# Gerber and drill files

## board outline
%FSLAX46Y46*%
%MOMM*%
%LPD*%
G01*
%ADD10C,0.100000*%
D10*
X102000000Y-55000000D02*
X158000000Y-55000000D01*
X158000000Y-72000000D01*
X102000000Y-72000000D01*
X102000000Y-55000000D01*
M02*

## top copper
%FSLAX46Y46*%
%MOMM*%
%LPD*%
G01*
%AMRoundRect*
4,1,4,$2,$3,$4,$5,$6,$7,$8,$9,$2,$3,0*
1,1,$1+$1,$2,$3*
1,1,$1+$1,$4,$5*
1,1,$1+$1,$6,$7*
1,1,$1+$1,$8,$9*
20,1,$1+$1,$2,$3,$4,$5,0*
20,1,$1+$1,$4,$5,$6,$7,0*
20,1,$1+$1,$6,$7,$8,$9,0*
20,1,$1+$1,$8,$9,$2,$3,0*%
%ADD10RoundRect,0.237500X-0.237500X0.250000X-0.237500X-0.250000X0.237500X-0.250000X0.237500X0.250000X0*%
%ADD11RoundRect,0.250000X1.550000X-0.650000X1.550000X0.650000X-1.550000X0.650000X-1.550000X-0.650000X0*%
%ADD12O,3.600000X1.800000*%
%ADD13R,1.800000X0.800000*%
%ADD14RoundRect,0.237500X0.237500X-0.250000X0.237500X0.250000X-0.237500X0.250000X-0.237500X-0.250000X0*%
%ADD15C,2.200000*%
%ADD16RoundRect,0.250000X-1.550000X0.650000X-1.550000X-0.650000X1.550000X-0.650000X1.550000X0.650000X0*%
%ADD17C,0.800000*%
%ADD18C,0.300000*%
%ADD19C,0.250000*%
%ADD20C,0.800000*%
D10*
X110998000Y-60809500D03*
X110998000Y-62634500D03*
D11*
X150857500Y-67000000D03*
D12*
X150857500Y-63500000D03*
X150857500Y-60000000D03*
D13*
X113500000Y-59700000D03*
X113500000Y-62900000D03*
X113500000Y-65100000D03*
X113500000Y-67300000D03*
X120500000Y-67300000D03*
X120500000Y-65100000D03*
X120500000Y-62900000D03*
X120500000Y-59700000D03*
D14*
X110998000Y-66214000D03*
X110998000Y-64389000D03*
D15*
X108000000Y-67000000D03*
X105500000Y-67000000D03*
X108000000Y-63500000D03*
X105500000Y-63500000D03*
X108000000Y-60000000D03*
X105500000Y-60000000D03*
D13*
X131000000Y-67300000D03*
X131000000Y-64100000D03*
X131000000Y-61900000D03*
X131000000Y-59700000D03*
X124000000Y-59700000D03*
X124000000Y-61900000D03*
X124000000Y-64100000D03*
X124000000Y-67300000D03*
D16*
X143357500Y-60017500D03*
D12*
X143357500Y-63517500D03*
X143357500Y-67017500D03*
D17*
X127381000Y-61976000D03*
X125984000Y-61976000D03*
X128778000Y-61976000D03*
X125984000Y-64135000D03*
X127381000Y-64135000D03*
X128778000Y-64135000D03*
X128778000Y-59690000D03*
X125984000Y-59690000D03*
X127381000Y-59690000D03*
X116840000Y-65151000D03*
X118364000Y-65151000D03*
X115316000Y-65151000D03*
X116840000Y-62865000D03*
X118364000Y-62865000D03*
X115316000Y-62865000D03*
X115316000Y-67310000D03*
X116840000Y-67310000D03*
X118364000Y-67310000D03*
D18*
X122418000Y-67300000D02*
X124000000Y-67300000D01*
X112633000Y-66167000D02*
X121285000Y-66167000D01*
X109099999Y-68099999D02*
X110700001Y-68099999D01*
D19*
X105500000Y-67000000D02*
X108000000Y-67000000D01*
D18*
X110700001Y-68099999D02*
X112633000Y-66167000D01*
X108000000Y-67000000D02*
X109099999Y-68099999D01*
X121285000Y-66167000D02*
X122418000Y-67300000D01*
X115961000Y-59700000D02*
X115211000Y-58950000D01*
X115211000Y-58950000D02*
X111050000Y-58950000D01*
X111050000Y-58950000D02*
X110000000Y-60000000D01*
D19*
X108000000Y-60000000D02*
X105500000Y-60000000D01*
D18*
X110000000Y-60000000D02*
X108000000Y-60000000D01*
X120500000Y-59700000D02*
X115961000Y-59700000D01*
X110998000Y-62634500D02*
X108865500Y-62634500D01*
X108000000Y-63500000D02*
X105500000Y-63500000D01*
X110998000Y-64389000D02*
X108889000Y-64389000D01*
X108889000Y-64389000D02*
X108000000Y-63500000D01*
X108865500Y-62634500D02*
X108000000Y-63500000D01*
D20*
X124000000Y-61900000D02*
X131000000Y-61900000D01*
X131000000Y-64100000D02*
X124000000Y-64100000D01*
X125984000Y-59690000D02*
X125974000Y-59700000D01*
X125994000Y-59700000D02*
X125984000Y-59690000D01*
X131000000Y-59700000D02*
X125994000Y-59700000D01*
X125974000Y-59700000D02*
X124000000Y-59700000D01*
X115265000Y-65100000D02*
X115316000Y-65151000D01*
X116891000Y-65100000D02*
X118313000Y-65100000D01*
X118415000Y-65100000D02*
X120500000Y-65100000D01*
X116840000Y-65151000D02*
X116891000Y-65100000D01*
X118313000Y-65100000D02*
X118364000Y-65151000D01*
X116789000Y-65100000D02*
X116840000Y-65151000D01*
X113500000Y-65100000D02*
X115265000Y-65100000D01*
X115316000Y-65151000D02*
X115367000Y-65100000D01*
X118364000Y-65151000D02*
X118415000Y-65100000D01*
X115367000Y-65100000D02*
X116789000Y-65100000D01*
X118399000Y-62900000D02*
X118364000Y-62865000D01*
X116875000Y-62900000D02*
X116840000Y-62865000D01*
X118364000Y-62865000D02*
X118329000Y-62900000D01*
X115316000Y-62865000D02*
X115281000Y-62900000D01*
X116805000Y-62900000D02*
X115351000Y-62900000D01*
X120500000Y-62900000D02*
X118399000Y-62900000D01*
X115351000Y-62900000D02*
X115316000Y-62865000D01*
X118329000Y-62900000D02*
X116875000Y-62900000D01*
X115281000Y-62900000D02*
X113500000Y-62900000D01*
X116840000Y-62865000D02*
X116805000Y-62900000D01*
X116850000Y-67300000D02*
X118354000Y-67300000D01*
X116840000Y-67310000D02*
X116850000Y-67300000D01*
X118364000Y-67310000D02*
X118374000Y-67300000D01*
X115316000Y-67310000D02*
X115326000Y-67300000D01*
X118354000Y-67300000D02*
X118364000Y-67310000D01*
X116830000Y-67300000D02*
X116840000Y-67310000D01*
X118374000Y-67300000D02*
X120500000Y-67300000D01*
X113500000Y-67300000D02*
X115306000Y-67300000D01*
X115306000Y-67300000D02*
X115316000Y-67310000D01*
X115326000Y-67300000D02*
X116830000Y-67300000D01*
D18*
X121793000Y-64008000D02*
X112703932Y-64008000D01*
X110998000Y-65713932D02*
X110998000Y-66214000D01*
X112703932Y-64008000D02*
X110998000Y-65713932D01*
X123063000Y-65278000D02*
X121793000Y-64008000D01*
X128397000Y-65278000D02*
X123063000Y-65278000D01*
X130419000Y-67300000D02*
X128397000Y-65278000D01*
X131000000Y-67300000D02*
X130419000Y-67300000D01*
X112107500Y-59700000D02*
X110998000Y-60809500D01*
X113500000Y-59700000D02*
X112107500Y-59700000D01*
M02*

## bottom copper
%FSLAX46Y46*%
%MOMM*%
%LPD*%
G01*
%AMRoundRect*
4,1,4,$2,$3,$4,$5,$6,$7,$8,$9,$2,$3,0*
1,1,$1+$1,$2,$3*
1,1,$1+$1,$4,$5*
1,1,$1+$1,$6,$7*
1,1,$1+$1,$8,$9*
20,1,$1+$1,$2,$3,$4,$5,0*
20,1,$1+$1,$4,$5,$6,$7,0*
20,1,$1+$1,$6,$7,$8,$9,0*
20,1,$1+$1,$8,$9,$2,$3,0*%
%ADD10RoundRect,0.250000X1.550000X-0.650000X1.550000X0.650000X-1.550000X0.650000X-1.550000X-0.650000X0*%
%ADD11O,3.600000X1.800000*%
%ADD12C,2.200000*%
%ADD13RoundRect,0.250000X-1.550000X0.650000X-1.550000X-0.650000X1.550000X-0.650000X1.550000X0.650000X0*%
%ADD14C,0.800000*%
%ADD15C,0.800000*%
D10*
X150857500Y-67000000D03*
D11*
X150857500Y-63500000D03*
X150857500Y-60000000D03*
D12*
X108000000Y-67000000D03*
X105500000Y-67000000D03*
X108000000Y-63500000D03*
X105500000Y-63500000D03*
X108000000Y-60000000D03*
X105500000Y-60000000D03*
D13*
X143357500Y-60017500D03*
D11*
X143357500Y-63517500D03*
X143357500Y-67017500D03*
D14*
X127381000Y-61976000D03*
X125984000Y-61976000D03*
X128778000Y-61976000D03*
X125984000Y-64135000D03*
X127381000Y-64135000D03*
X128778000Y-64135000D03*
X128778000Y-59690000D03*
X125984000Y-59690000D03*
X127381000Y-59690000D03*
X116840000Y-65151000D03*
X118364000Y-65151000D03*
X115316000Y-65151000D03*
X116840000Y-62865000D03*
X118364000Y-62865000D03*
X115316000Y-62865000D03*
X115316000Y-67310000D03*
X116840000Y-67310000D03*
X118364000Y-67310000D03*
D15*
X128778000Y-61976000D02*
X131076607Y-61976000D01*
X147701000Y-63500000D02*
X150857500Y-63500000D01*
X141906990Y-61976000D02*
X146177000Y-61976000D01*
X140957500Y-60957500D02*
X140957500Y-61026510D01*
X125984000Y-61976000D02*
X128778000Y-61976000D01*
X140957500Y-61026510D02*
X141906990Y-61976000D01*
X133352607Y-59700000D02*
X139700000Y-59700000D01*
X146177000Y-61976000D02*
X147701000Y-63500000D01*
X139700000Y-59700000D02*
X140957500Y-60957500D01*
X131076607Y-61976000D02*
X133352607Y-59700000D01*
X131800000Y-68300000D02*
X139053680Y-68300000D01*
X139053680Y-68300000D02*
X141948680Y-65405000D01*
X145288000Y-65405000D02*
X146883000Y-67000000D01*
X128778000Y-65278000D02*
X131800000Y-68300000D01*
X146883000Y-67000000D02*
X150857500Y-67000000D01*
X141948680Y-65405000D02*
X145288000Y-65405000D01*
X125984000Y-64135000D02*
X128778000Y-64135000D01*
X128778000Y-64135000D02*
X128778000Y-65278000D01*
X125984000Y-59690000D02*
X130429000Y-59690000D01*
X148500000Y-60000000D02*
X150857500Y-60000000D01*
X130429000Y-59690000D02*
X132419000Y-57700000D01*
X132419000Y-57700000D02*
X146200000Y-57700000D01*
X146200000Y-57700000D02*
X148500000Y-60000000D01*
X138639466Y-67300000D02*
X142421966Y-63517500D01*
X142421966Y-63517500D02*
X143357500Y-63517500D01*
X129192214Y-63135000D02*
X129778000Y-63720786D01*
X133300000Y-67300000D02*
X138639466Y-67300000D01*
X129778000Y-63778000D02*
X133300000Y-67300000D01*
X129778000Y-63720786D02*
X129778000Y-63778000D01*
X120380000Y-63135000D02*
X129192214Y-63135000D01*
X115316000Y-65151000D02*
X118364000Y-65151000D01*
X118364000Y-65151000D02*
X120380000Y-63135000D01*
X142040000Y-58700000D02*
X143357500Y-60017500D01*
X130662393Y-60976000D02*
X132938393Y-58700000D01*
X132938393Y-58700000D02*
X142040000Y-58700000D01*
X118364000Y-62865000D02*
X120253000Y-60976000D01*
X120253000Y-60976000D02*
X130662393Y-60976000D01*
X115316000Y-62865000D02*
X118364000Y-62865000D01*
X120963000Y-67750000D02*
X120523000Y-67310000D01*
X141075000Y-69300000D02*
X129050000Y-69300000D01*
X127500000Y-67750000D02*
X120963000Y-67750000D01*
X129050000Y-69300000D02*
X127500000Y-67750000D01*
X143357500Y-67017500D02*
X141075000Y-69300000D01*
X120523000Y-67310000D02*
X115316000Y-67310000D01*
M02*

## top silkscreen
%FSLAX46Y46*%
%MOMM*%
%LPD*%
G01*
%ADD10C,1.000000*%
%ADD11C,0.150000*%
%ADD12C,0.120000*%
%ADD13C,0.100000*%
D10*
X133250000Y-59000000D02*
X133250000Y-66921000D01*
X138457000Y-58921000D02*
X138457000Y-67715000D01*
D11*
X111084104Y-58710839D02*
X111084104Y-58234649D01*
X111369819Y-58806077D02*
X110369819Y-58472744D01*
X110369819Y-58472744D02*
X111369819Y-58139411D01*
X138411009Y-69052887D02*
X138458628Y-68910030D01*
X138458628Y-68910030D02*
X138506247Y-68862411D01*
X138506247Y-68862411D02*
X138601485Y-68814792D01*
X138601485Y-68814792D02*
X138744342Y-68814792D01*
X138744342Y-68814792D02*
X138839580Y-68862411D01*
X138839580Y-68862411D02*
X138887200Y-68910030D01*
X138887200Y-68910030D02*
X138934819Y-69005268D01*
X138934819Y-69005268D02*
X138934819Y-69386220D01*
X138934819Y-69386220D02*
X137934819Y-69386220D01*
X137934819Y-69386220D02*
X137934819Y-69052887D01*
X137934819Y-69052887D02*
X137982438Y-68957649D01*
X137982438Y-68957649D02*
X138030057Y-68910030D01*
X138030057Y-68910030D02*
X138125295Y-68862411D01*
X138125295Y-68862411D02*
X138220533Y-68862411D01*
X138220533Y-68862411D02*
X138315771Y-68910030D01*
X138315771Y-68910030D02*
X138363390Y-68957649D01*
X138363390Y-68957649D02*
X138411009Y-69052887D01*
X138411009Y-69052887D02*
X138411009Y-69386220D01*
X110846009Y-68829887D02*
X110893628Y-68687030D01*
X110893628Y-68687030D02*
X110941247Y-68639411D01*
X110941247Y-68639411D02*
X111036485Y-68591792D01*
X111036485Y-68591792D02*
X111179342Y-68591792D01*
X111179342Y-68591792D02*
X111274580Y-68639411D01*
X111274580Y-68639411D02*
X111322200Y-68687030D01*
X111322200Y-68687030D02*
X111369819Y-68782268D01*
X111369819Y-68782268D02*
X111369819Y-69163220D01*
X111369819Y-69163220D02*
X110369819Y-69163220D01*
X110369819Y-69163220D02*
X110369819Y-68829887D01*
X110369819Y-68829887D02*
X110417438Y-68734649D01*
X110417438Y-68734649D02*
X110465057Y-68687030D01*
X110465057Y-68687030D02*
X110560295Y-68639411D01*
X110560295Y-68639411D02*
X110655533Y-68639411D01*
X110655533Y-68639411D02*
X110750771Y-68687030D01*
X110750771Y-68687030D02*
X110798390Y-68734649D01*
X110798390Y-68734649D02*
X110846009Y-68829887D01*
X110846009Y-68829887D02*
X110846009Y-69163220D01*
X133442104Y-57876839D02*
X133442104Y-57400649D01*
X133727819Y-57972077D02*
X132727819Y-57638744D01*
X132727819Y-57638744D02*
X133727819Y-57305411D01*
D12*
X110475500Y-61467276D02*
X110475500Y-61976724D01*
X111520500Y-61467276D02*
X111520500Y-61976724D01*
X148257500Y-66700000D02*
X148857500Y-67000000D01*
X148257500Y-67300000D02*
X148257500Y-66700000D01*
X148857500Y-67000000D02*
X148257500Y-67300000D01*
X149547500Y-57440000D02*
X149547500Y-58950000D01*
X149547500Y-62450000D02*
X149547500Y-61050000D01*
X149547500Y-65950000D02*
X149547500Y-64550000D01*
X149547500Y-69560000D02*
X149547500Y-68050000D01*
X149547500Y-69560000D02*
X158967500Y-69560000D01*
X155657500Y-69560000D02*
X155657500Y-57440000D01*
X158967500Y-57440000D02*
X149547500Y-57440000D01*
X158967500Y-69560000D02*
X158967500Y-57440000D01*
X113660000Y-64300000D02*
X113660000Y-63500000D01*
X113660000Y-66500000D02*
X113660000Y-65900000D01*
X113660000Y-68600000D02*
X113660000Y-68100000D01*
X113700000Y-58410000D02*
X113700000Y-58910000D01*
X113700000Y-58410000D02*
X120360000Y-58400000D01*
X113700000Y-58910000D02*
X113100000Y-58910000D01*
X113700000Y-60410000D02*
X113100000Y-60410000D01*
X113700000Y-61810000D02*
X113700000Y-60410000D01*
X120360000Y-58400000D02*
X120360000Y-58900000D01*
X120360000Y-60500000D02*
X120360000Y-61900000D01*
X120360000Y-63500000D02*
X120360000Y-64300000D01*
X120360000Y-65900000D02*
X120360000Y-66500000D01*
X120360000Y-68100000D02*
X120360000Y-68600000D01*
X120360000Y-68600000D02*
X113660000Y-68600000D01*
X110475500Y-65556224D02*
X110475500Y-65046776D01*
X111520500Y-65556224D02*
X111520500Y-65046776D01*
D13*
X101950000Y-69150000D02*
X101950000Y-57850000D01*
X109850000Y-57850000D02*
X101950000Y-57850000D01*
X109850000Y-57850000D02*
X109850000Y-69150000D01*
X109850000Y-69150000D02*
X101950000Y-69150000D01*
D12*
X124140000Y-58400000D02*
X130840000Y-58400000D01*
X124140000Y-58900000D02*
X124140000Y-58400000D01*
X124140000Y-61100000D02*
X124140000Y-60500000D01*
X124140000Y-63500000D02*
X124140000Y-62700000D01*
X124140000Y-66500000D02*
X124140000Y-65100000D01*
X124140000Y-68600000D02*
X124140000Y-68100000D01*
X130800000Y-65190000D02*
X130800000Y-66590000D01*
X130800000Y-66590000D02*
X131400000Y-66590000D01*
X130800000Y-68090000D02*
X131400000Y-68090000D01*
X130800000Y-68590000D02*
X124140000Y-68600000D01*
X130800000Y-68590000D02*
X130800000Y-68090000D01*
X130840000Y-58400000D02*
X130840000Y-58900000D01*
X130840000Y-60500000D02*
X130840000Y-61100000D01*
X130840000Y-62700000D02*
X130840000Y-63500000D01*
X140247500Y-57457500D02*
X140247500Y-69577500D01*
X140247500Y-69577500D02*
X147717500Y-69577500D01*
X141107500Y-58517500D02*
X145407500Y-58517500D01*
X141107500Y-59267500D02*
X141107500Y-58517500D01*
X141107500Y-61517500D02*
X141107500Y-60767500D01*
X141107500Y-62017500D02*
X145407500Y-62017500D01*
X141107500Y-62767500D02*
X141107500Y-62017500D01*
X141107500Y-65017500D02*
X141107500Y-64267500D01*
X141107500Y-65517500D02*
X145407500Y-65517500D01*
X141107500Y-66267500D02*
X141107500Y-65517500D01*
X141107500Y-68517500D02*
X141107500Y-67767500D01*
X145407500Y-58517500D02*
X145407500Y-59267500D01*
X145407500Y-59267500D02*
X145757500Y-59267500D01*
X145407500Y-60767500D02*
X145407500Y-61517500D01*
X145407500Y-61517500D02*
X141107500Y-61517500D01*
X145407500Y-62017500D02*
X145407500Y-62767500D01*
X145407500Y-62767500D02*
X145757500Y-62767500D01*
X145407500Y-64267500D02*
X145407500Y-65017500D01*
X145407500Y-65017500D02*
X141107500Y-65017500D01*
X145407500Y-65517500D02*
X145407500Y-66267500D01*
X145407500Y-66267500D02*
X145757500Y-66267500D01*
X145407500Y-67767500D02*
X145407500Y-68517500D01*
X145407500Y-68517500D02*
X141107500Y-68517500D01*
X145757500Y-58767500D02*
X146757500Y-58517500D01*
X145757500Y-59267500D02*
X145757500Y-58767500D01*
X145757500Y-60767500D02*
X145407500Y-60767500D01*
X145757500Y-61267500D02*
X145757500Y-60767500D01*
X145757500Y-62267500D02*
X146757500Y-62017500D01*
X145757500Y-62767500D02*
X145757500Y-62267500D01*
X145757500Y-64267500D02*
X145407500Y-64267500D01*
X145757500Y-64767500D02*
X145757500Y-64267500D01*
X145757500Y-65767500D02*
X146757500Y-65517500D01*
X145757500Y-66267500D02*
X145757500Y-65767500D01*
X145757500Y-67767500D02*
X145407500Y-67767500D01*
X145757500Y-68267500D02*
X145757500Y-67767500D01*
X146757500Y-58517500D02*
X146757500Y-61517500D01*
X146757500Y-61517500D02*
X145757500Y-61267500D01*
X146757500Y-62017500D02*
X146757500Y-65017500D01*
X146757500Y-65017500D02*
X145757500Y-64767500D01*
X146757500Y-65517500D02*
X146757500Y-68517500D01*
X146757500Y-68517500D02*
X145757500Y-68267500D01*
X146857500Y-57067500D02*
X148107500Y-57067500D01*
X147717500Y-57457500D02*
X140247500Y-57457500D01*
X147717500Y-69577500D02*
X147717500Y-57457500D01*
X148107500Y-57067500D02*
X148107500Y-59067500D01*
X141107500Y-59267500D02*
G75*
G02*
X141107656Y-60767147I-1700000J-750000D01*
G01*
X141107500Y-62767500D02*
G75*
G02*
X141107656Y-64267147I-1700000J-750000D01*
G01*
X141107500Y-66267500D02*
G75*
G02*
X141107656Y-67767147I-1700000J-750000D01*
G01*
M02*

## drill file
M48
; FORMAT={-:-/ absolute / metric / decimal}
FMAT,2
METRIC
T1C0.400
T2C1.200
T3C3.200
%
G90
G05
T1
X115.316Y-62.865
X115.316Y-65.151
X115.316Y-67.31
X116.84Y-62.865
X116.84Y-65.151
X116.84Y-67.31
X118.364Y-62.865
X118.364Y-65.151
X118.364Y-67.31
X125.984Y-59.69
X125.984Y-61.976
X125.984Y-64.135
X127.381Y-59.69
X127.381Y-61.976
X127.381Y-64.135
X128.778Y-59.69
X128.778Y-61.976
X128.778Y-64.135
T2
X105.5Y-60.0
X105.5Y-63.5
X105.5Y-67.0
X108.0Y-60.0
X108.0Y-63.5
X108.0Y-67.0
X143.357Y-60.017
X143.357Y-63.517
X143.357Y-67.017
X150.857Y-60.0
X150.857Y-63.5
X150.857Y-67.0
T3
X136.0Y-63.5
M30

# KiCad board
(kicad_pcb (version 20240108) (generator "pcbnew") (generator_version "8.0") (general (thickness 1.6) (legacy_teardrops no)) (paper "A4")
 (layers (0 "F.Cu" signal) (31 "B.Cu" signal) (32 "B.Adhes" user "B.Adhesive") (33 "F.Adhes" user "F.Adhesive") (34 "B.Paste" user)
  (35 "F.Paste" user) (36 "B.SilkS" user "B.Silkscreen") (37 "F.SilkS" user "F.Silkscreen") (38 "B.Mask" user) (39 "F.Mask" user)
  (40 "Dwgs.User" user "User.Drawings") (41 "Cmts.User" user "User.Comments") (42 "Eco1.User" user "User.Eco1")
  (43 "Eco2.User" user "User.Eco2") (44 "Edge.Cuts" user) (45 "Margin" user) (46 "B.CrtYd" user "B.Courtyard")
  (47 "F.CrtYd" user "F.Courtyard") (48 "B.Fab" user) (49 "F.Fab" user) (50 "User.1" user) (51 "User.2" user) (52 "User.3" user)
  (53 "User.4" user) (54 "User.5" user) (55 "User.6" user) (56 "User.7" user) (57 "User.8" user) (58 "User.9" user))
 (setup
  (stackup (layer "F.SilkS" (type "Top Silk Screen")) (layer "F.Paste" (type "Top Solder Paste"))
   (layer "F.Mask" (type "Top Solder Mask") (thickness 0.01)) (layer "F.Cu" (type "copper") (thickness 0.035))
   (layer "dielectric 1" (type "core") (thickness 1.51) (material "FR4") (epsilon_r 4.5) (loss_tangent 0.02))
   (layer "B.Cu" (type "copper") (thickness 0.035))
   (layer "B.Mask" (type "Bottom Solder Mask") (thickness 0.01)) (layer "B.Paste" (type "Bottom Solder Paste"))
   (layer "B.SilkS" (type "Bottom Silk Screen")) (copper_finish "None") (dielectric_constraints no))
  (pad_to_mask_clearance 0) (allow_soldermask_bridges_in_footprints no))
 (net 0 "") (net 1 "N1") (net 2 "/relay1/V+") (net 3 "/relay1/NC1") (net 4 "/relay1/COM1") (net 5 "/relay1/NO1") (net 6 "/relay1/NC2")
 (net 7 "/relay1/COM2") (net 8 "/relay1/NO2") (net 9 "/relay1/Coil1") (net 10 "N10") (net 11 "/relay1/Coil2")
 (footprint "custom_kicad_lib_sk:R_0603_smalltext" (layer "F.Cu") (at 110.998 61.722 -90)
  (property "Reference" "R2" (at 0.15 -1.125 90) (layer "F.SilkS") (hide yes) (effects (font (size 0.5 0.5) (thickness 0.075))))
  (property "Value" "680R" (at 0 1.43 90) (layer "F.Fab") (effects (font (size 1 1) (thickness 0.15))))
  (fp_line (start -0.254724 0.5225) (end 0.254724 0.5225) (stroke (width 0.12) (type solid)) (layer "F.SilkS"))
  (fp_line (start -0.254724 -0.5225) (end 0.254724 -0.5225) (stroke (width 0.12) (type solid)) (layer "F.SilkS"))
  (pad "1" smd roundrect (at -0.9125 0 270) (size 0.975 0.95) (layers "F.Cu" "F.Paste" "F.Mask") (roundrect_rratio 0.25) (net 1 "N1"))
  (pad "2" smd roundrect (at 0.9125 0 270) (size 0.975 0.95) (layers "F.Cu" "F.Paste" "F.Mask") (roundrect_rratio 0.25) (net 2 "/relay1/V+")))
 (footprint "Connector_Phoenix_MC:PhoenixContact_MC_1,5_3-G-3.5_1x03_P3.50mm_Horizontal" (layer "F.Cu") (at 150.8575 67 90)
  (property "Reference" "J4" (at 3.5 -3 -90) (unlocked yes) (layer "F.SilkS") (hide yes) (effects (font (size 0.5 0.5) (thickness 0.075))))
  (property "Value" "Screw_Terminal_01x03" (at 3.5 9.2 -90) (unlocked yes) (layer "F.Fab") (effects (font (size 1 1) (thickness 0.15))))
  (fp_line (start 0.3 -2.6) (end 0 -2) (stroke (width 0.12) (type solid)) (layer "F.SilkS"))
  (fp_line (start -0.3 -2.6) (end 0.3 -2.6) (stroke (width 0.12) (type solid)) (layer "F.SilkS"))
  (fp_line (start 0 -2) (end -0.3 -2.6) (stroke (width 0.12) (type solid)) (layer "F.SilkS"))
  (fp_line (start 9.56 -1.31) (end 8.05 -1.31) (stroke (width 0.12) (type solid)) (layer "F.SilkS"))
  (fp_line (start 4.55 -1.31) (end 5.95 -1.31) (stroke (width 0.12) (type solid)) (layer "F.SilkS"))
  (fp_line (start 1.05 -1.31) (end 2.45 -1.31) (stroke (width 0.12) (type solid)) (layer "F.SilkS"))
  (fp_line (start -2.56 -1.31) (end -1.05 -1.31) (stroke (width 0.12) (type solid)) (layer "F.SilkS"))
  (fp_line (start -2.56 -1.31) (end -2.56 8.11) (stroke (width 0.12) (type solid)) (layer "F.SilkS"))
  (fp_line (start -2.56 4.8) (end 9.56 4.8) (stroke (width 0.12) (type solid)) (layer "F.SilkS"))
  (fp_line (start 9.56 8.11) (end 9.56 -1.31) (stroke (width 0.12) (type solid)) (layer "F.SilkS"))
  (fp_line (start -2.56 8.11) (end 9.56 8.11) (stroke (width 0.12) (type solid)) (layer "F.SilkS"))
  (pad "1" thru_hole roundrect (at 0 0 90) (size 1.8 3.6) (drill 1.2) (layers "*.Cu" "*.Mask") (remove_unused_layers no)
   (roundrect_rratio 0.138889) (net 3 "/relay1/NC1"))
  (pad "2" thru_hole oval (at 3.5 0 90) (size 1.8 3.6) (drill 1.2) (layers "*.Cu" "*.Mask") (remove_unused_layers no) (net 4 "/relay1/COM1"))
  (pad "3" thru_hole oval (at 7 0 90) (size 1.8 3.6) (drill 1.2) (layers "*.Cu" "*.Mask") (remove_unused_layers no) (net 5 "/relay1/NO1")))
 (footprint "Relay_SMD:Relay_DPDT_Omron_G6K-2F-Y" (layer "F.Cu") (at 117 63.5)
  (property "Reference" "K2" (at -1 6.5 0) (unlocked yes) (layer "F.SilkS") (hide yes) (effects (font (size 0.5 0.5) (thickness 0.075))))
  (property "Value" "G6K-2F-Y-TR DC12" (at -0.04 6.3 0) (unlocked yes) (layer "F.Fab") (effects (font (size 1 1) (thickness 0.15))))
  (fp_line (start -3.34 0.8) (end -3.34 0) (stroke (width 0.12) (type solid)) (layer "F.SilkS"))
  (fp_line (start -3.34 3) (end -3.34 2.4) (stroke (width 0.12) (type solid)) (layer "F.SilkS"))
  (fp_line (start -3.34 5.1) (end -3.34 4.6) (stroke (width 0.12) (type solid)) (layer "F.SilkS"))
  (fp_line (start -3.3 -5.09) (end -3.3 -4.59) (stroke (width 0.12) (type solid)) (layer "F.SilkS"))
  (fp_line (start -3.3 -5.09) (end 3.36 -5.1) (stroke (width 0.12) (type solid)) (layer "F.SilkS"))
  (fp_line (start -3.3 -4.59) (end -3.9 -4.59) (stroke (width 0.12) (type solid)) (layer "F.SilkS"))
  (fp_line (start -3.3 -3.09) (end -3.9 -3.09) (stroke (width 0.12) (type solid)) (layer "F.SilkS"))
  (fp_line (start -3.3 -1.69) (end -3.3 -3.09) (stroke (width 0.12) (type solid)) (layer "F.SilkS"))
  (fp_line (start 3.36 -5.1) (end 3.36 -4.6) (stroke (width 0.12) (type solid)) (layer "F.SilkS"))
  (fp_line (start 3.36 -3) (end 3.36 -1.6) (stroke (width 0.12) (type solid)) (layer "F.SilkS"))
  (fp_line (start 3.36 0) (end 3.36 0.8) (stroke (width 0.12) (type solid)) (layer "F.SilkS"))
  (fp_line (start 3.36 2.4) (end 3.36 3) (stroke (width 0.12) (type solid)) (layer "F.SilkS"))
  (fp_line (start 3.36 4.6) (end 3.36 5.1) (stroke (width 0.12) (type solid)) (layer "F.SilkS"))
  (fp_line (start 3.36 5.1) (end -3.34 5.1) (stroke (width 0.12) (type solid)) (layer "F.SilkS"))
  (pad "1" smd rect (at -3.5 -3.8) (size 1.8 0.8) (layers "F.Cu" "F.Paste" "F.Mask") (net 1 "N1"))
  (pad "2" smd rect (at -3.5 -0.6) (size 1.8 0.8) (layers "F.Cu" "F.Paste" "F.Mask") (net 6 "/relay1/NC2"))
  (pad "3" smd rect (at -3.5 1.6) (size 1.8 0.8) (layers "F.Cu" "F.Paste" "F.Mask") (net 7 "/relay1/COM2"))
  (pad "4" smd rect (at -3.5 3.8) (size 1.8 0.8) (layers "F.Cu" "F.Paste" "F.Mask") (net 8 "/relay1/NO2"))
  (pad "5" smd rect (at 3.5 3.8) (size 1.8 0.8) (layers "F.Cu" "F.Paste" "F.Mask") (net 8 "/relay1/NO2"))
  (pad "6" smd rect (at 3.5 1.6) (size 1.8 0.8) (layers "F.Cu" "F.Paste" "F.Mask") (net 7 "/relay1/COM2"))
  (pad "7" smd rect (at 3.5 -0.6) (size 1.8 0.8) (layers "F.Cu" "F.Paste" "F.Mask") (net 6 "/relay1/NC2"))
  (pad "8" smd rect (at 3.5 -3.8) (size 1.8 0.8) (layers "F.Cu" "F.Paste" "F.Mask") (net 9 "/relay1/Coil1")))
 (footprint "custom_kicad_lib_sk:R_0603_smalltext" (layer "F.Cu") (at 110.998 65.3015 90)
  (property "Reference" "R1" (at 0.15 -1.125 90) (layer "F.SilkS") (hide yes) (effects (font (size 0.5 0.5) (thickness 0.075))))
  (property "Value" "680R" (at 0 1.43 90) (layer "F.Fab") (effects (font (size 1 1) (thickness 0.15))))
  (fp_line (start -0.254724 -0.5225) (end 0.254724 -0.5225) (stroke (width 0.12) (type solid)) (layer "F.SilkS"))
  (fp_line (start -0.254724 0.5225) (end 0.254724 0.5225) (stroke (width 0.12) (type solid)) (layer "F.SilkS"))
  (pad "1" smd roundrect (at -0.9125 0 90) (size 0.975 0.95) (layers "F.Cu" "F.Paste" "F.Mask") (roundrect_rratio 0.25) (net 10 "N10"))
  (pad "2" smd roundrect (at 0.9125 0 90) (size 0.975 0.95) (layers "F.Cu" "F.Paste" "F.Mask") (roundrect_rratio 0.25) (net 2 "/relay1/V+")))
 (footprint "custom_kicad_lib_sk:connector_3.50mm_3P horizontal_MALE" (layer "F.Cu") (at 108 63.5 -90)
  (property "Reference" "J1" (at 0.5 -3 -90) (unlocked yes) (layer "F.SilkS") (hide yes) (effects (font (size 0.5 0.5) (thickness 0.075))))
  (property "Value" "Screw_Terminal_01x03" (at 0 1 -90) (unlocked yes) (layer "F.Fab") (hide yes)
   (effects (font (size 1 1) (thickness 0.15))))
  (fp_line (start 5.65 6.05) (end -5.65 6.05) (stroke (width 0.1) (type default)) (layer "F.SilkS"))
  (fp_line (start -5.65 -1.85) (end -5.65 6.05) (stroke (width 0.1) (type default)) (layer "F.SilkS"))
  (fp_line (start -5.65 -1.85) (end 5.65 -1.85) (stroke (width 0.1) (type default)) (layer "F.SilkS"))
  (fp_line (start 5.65 -1.85) (end 5.65 6.05) (stroke (width 0.1) (type default)) (layer "F.SilkS"))
  (pad "1" thru_hole circle (at 3.5 0 270) (size 2.2 2.2) (drill 1.2) (layers "*.Cu" "*.Mask") (remove_unused_layers no)
   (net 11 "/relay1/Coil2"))
  (pad "1" thru_hole circle (at 3.5 2.5 270) (size 2.2 2.2) (drill 1.2) (layers "*.Cu" "*.Mask") (remove_unused_layers no)
   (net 11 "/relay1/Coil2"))
  (pad "2" thru_hole circle (at 0 0 270) (size 2.2 2.2) (drill 1.2) (layers "*.Cu" "*.Mask") (remove_unused_layers no) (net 2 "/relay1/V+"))
  (pad "2" thru_hole circle (at 0 2.5 270) (size 2.2 2.2) (drill 1.2) (layers "*.Cu" "*.Mask") (remove_unused_layers no)
   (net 2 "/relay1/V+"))
  (pad "3" thru_hole circle (at -3.5 0 270) (size 2.2 2.2) (drill 1.2) (layers "*.Cu" "*.Mask") (remove_unused_layers no)
   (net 9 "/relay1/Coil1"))
  (pad "3" thru_hole circle (at -3.5 2.5 270) (size 2.2 2.2) (drill 1.2) (layers "*.Cu" "*.Mask") (remove_unused_layers no)
   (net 9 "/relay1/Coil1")))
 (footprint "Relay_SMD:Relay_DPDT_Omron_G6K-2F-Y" (layer "F.Cu") (at 127.5 63.5 180)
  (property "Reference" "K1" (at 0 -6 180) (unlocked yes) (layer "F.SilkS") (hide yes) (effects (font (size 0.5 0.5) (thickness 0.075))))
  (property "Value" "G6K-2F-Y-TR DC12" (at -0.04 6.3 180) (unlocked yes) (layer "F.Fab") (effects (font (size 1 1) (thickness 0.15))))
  (fp_line (start 3.36 5.1) (end -3.34 5.1) (stroke (width 0.12) (type solid)) (layer "F.SilkS"))
  (fp_line (start 3.36 4.6) (end 3.36 5.1) (stroke (width 0.12) (type solid)) (layer "F.SilkS"))
  (fp_line (start 3.36 2.4) (end 3.36 3) (stroke (width 0.12) (type solid)) (layer "F.SilkS"))
  (fp_line (start 3.36 0) (end 3.36 0.8) (stroke (width 0.12) (type solid)) (layer "F.SilkS"))
  (fp_line (start 3.36 -3) (end 3.36 -1.6) (stroke (width 0.12) (type solid)) (layer "F.SilkS"))
  (fp_line (start 3.36 -5.1) (end 3.36 -4.6) (stroke (width 0.12) (type solid)) (layer "F.SilkS"))
  (fp_line (start -3.3 -1.69) (end -3.3 -3.09) (stroke (width 0.12) (type solid)) (layer "F.SilkS"))
  (fp_line (start -3.3 -3.09) (end -3.9 -3.09) (stroke (width 0.12) (type solid)) (layer "F.SilkS"))
  (fp_line (start -3.3 -4.59) (end -3.9 -4.59) (stroke (width 0.12) (type solid)) (layer "F.SilkS"))
  (fp_line (start -3.3 -5.09) (end 3.36 -5.1) (stroke (width 0.12) (type solid)) (layer "F.SilkS"))
  (fp_line (start -3.3 -5.09) (end -3.3 -4.59) (stroke (width 0.12) (type solid)) (layer "F.SilkS"))
  (fp_line (start -3.34 5.1) (end -3.34 4.6) (stroke (width 0.12) (type solid)) (layer "F.SilkS"))
  (fp_line (start -3.34 3) (end -3.34 2.4) (stroke (width 0.12) (type solid)) (layer "F.SilkS"))
  (fp_line (start -3.34 0.8) (end -3.34 0) (stroke (width 0.12) (type solid)) (layer "F.SilkS"))
  (pad "1" smd rect (at -3.5 -3.8 180) (size 1.8 0.8) (layers "F.Cu" "F.Paste" "F.Mask") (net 10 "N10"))
  (pad "2" smd rect (at -3.5 -0.6 180) (size 1.8 0.8) (layers "F.Cu" "F.Paste" "F.Mask") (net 3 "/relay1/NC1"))
  (pad "3" smd rect (at -3.5 1.6 180) (size 1.8 0.8) (layers "F.Cu" "F.Paste" "F.Mask") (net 4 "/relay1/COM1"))
  (pad "4" smd rect (at -3.5 3.8 180) (size 1.8 0.8) (layers "F.Cu" "F.Paste" "F.Mask") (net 5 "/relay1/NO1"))
  (pad "5" smd rect (at 3.5 3.8 180) (size 1.8 0.8) (layers "F.Cu" "F.Paste" "F.Mask") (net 5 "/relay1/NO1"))
  (pad "6" smd rect (at 3.5 1.6 180) (size 1.8 0.8) (layers "F.Cu" "F.Paste" "F.Mask") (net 4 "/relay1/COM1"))
  (pad "7" smd rect (at 3.5 -0.6 180) (size 1.8 0.8) (layers "F.Cu" "F.Paste" "F.Mask") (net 3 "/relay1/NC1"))
  (pad "8" smd rect (at 3.5 -3.8 180) (size 1.8 0.8) (layers "F.Cu" "F.Paste" "F.Mask") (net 11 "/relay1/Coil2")))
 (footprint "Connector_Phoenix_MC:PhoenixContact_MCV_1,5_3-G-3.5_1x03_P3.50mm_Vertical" (layer "F.Cu") (at 143.3575 60.0175 -90)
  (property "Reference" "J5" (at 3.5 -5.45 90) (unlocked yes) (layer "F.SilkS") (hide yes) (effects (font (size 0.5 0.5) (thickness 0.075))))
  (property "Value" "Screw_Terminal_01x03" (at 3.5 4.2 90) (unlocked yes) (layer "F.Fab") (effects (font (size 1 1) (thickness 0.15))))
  (fp_line (start -2.56 3.11) (end 9.56 3.11) (stroke (width 0.12) (type solid)) (layer "F.SilkS"))
  (fp_line (start 9.56 3.11) (end 9.56 -4.36) (stroke (width 0.12) (type solid)) (layer "F.SilkS"))
  (fp_line (start -1.5 2.25) (end -1.5 -2.05) (stroke (width 0.12) (type solid)) (layer "F.SilkS"))
  (fp_line (start -0.75 2.25) (end -1.5 2.25) (stroke (width 0.12) (type solid)) (layer "F.SilkS"))
  (fp_line (start 1.5 2.25) (end 0.75 2.25) (stroke (width 0.12) (type solid)) (layer "F.SilkS"))
  (fp_line (start 2 2.25) (end 2 -2.05) (stroke (width 0.12) (type solid)) (layer "F.SilkS"))
  (fp_line (start 2.75 2.25) (end 2 2.25) (stroke (width 0.12) (type solid)) (layer "F.SilkS"))
  (fp_line (start 5 2.25) (end 4.25 2.25) (stroke (width 0.12) (type solid)) (layer "F.SilkS"))
  (fp_line (start 5.5 2.25) (end 5.5 -2.05) (stroke (width 0.12) (type solid)) (layer "F.SilkS"))
  (fp_line (start 6.25 2.25) (end 5.5 2.25) (stroke (width 0.12) (type solid)) (layer "F.SilkS"))
  (fp_line (start 8.5 2.25) (end 7.75 2.25) (stroke (width 0.12) (type solid)) (layer "F.SilkS"))
  (fp_line (start -1.5 -2.05) (end -0.75 -2.05) (stroke (width 0.12) (type solid)) (layer "F.SilkS"))
  (fp_line (start -0.75 -2.05) (end -0.75 -2.4) (stroke (width 0.12) (type solid)) (layer "F.SilkS"))
  (fp_line (start 0.75 -2.05) (end 1.5 -2.05) (stroke (width 0.12) (type solid)) (layer "F.SilkS"))
  (fp_line (start 1.5 -2.05) (end 1.5 2.25) (stroke (width 0.12) (type solid)) (layer "F.SilkS"))
  (fp_line (start 2 -2.05) (end 2.75 -2.05) (stroke (width 0.12) (type solid)) (layer "F.SilkS"))
  (fp_line (start 2.75 -2.05) (end 2.75 -2.4) (stroke (width 0.12) (type solid)) (layer "F.SilkS"))
  (fp_line (start 4.25 -2.05) (end 5 -2.05) (stroke (width 0.12) (type solid)) (layer "F.SilkS"))
  (fp_line (start 5 -2.05) (end 5 2.25) (stroke (width 0.12) (type solid)) (layer "F.SilkS"))
  (fp_line (start 5.5 -2.05) (end 6.25 -2.05) (stroke (width 0.12) (type solid)) (layer "F.SilkS"))
  (fp_line (start 6.25 -2.05) (end 6.25 -2.4) (stroke (width 0.12) (type solid)) (layer "F.SilkS"))
  (fp_line (start 7.75 -2.05) (end 8.5 -2.05) (stroke (width 0.12) (type solid)) (layer "F.SilkS"))
  (fp_line (start 8.5 -2.05) (end 8.5 2.25) (stroke (width 0.12) (type solid)) (layer "F.SilkS"))
  (fp_line (start -1.25 -2.4) (end -1.5 -3.4) (stroke (width 0.12) (type solid)) (layer "F.SilkS"))
  (fp_line (start -0.75 -2.4) (end -1.25 -2.4) (stroke (width 0.12) (type solid)) (layer "F.SilkS"))
  (fp_line (start 0.75 -2.4) (end 0.75 -2.05) (stroke (width 0.12) (type solid)) (layer "F.SilkS"))
  (fp_line (start 1.25 -2.4) (end 0.75 -2.4) (stroke (width 0.12) (type solid)) (layer "F.SilkS"))
  (fp_line (start 2.25 -2.4) (end 2 -3.4) (stroke (width 0.12) (type solid)) (layer "F.SilkS"))
  (fp_line (start 2.75 -2.4) (end 2.25 -2.4) (stroke (width 0.12) (type solid)) (layer "F.SilkS"))
  (fp_line (start 4.25 -2.4) (end 4.25 -2.05) (stroke (width 0.12) (type solid)) (layer "F.SilkS"))
  (fp_line (start 4.75 -2.4) (end 4.25 -2.4) (stroke (width 0.12) (type solid)) (layer "F.SilkS"))
  (fp_line (start 5.75 -2.4) (end 5.5 -3.4) (stroke (width 0.12) (type solid)) (layer "F.SilkS"))
  (fp_line (start 6.25 -2.4) (end 5.75 -2.4) (stroke (width 0.12) (type solid)) (layer "F.SilkS"))
  (fp_line (start 7.75 -2.4) (end 7.75 -2.05) (stroke (width 0.12) (type solid)) (layer "F.SilkS"))
  (fp_line (start 8.25 -2.4) (end 7.75 -2.4) (stroke (width 0.12) (type solid)) (layer "F.SilkS"))
  (fp_line (start -1.5 -3.4) (end 1.5 -3.4) (stroke (width 0.12) (type solid)) (layer "F.SilkS"))
  (fp_line (start 1.5 -3.4) (end 1.25 -2.4) (stroke (width 0.12) (type solid)) (layer "F.SilkS"))
  (fp_line (start 2 -3.4) (end 5 -3.4) (stroke (width 0.12) (type solid)) (layer "F.SilkS"))
  (fp_line (start 5 -3.4) (end 4.75 -2.4) (stroke (width 0.12) (type solid)) (layer "F.SilkS"))
  (fp_line (start 5.5 -3.4) (end 8.5 -3.4) (stroke (width 0.12) (type solid)) (layer "F.SilkS"))
  (fp_line (start 8.5 -3.4) (end 8.25 -2.4) (stroke (width 0.12) (type solid)) (layer "F.SilkS"))
  (fp_line (start -2.95 -3.5) (end -2.95 -4.75) (stroke (width 0.12) (type solid)) (layer "F.SilkS"))
  (fp_line (start -2.56 -4.36) (end -2.56 3.11) (stroke (width 0.12) (type solid)) (layer "F.SilkS"))
  (fp_line (start 9.56 -4.36) (end -2.56 -4.36) (stroke (width 0.12) (type solid)) (layer "F.SilkS"))
  (fp_line (start -2.95 -4.75) (end -0.95 -4.75) (stroke (width 0.12) (type solid)) (layer "F.SilkS"))
  (fp_arc (start -0.75 2.25) (mid -0.000193 2.09191) (end 0.749647 2.249844) (stroke (width 0.12) (type solid)) (layer "F.SilkS"))
  (fp_arc (start 2.75 2.25) (mid 3.499807 2.09191) (end 4.249647 2.249844) (stroke (width 0.12) (type solid)) (layer "F.SilkS"))
  (fp_arc (start 6.25 2.25) (mid 6.999807 2.09191) (end 7.749647 2.249844) (stroke (width 0.12) (type solid)) (layer "F.SilkS"))
  (pad "1" thru_hole roundrect (at 0 0 270) (size 1.8 3.6) (drill 1.2) (layers "*.Cu" "*.Mask") (remove_unused_layers no)
   (roundrect_rratio 0.138889) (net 6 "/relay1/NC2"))
  (pad "2" thru_hole oval (at 3.5 0 270) (size 1.8 3.6) (drill 1.2) (layers "*.Cu" "*.Mask") (remove_unused_layers no)
   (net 7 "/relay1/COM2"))
  (pad "3" thru_hole oval (at 7 0 270) (size 1.8 3.6) (drill 1.2) (layers "*.Cu" "*.Mask") (remove_unused_layers no) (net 8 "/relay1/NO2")))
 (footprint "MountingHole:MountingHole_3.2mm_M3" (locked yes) (layer "F.Cu") (at 136 63.5)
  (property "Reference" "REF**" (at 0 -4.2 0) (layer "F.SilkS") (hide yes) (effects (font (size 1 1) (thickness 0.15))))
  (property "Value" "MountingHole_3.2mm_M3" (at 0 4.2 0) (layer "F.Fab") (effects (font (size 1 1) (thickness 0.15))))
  (pad "" np_thru_hole circle (at 0 0) (size 3.2 3.2) (drill 3.2) (layers "*.Cu" "*.Mask")))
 (gr_line (start 133.25 59) (end 133.25 66.921) (stroke (width 1) (type default)) (layer "F.SilkS"))
 (gr_line (start 138.457 58.921) (end 138.457 67.715) (stroke (width 1) (type default)) (layer "F.SilkS"))
 (gr_rect (start 102 55) (end 158 72) (stroke (width 0.1) (type default)) (fill none) (layer "Edge.Cuts"))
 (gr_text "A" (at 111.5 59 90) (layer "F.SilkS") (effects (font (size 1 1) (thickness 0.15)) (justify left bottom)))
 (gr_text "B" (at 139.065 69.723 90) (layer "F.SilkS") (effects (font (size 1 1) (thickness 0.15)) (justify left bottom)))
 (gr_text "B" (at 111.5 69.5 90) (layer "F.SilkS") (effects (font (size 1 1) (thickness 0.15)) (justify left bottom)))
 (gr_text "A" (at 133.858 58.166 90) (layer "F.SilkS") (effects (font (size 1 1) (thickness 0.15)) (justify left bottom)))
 (segment (start 122.418 67.3) (end 124 67.3) (width 0.3) (layer "F.Cu") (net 11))
 (segment (start 112.633 66.167) (end 121.285 66.167) (width 0.3) (layer "F.Cu") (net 11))
 (segment (start 109.099999 68.099999) (end 110.700001 68.099999) (width 0.3) (layer "F.Cu") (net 11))
 (segment (start 105.5 67) (end 108 67) (width 0.25) (layer "F.Cu") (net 11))
 (segment (start 110.700001 68.099999) (end 112.633 66.167) (width 0.3) (layer "F.Cu") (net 11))
 (segment (start 108 67) (end 109.099999 68.099999) (width 0.3) (layer "F.Cu") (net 11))
 (segment (start 121.285 66.167) (end 122.418 67.3) (width 0.3) (layer "F.Cu") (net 11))
 (segment (start 115.961 59.7) (end 115.211 58.95) (width 0.3) (layer "F.Cu") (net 9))
 (segment (start 115.211 58.95) (end 111.05 58.95) (width 0.3) (layer "F.Cu") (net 9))
 (segment (start 111.05 58.95) (end 110 60) (width 0.3) (layer "F.Cu") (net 9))
 (segment (start 108 60) (end 105.5 60) (width 0.25) (layer "F.Cu") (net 9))
 (segment (start 110 60) (end 108 60) (width 0.3) (layer "F.Cu") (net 9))
 (segment (start 120.5 59.7) (end 115.961 59.7) (width 0.3) (layer "F.Cu") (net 9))
 (segment (start 110.998 62.6345) (end 108.8655 62.6345) (width 0.3) (layer "F.Cu") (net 2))
 (segment (start 108 63.5) (end 105.5 63.5) (width 0.3) (layer "F.Cu") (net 2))
 (segment (start 110.998 64.389) (end 108.889 64.389) (width 0.3) (layer "F.Cu") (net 2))
 (segment (start 108.889 64.389) (end 108 63.5) (width 0.3) (layer "F.Cu") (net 2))
 (segment (start 108.8655 62.6345) (end 108 63.5) (width 0.3) (layer "F.Cu") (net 2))
 (segment (start 124 61.9) (end 131 61.9) (width 0.8) (layer "F.Cu") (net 4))
 (via (at 127.381 61.976) (size 0.8) (drill 0.4) (layers "F.Cu" "B.Cu") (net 4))
 (via (at 125.984 61.976) (size 0.8) (drill 0.4) (layers "F.Cu" "B.Cu") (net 4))
 (via (at 128.778 61.976) (size 0.8) (drill 0.4) (layers "F.Cu" "B.Cu") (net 4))
 (segment (start 128.778 61.976) (end 131.076607 61.976) (width 0.8) (layer "B.Cu") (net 4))
 (segment (start 147.701 63.5) (end 150.8575 63.5) (width 0.8) (layer "B.Cu") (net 4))
 (segment (start 141.90699 61.976) (end 146.177 61.976) (width 0.8) (layer "B.Cu") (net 4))
 (segment (start 140.9575 60.9575) (end 140.9575 61.02651) (width 0.8) (layer "B.Cu") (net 4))
 (segment (start 125.984 61.976) (end 128.778 61.976) (width 0.8) (layer "B.Cu") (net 4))
 (segment (start 140.9575 61.02651) (end 141.90699 61.976) (width 0.8) (layer "B.Cu") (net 4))
 (segment (start 133.352607 59.7) (end 139.7 59.7) (width 0.8) (layer "B.Cu") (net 4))
 (segment (start 146.177 61.976) (end 147.701 63.5) (width 0.8) (layer "B.Cu") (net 4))
 (segment (start 139.7 59.7) (end 140.9575 60.9575) (width 0.8) (layer "B.Cu") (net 4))
 (segment (start 131.076607 61.976) (end 133.352607 59.7) (width 0.8) (layer "B.Cu") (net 4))
 (segment (start 131 64.1) (end 124 64.1) (width 0.8) (layer "F.Cu") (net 3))
 (via (at 125.984 64.135) (size 0.8) (drill 0.4) (layers "F.Cu" "B.Cu") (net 3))
 (via (at 127.381 64.135) (size 0.8) (drill 0.4) (layers "F.Cu" "B.Cu") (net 3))
 (via (at 128.778 64.135) (size 0.8) (drill 0.4) (layers "F.Cu" "B.Cu") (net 3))
 (segment (start 131.8 68.3) (end 139.05368 68.3) (width 0.8) (layer "B.Cu") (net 3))
 (segment (start 139.05368 68.3) (end 141.94868 65.405) (width 0.8) (layer "B.Cu") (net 3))
 (segment (start 145.288 65.405) (end 146.883 67) (width 0.8) (layer "B.Cu") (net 3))
 (segment (start 128.778 65.278) (end 131.8 68.3) (width 0.8) (layer "B.Cu") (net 3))
 (segment (start 146.883 67) (end 150.8575 67) (width 0.8) (layer "B.Cu") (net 3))
 (segment (start 141.94868 65.405) (end 145.288 65.405) (width 0.8) (layer "B.Cu") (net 3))
 (segment (start 125.984 64.135) (end 128.778 64.135) (width 0.8) (layer "B.Cu") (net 3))
 (segment (start 128.778 64.135) (end 128.778 65.278) (width 0.8) (layer "B.Cu") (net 3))
 (segment (start 125.984 59.69) (end 125.974 59.7) (width 0.8) (layer "F.Cu") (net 5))
 (segment (start 125.994 59.7) (end 125.984 59.69) (width 0.8) (layer "F.Cu") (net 5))
 (segment (start 131 59.7) (end 125.994 59.7) (width 0.8) (layer "F.Cu") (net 5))
 (segment (start 125.974 59.7) (end 124 59.7) (width 0.8) (layer "F.Cu") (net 5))
 (via (at 128.778 59.69) (size 0.8) (drill 0.4) (layers "F.Cu" "B.Cu") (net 5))
 (via (at 125.984 59.69) (size 0.8) (drill 0.4) (layers "F.Cu" "B.Cu") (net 5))
 (via (at 127.381 59.69) (size 0.8) (drill 0.4) (layers "F.Cu" "B.Cu") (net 5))
 (segment (start 125.984 59.69) (end 130.429 59.69) (width 0.8) (layer "B.Cu") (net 5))
 (segment (start 148.5 60) (end 150.8575 60) (width 0.8) (layer "B.Cu") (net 5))
 (segment (start 130.429 59.69) (end 132.419 57.7) (width 0.8) (layer "B.Cu") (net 5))
 (segment (start 132.419 57.7) (end 146.2 57.7) (width 0.8) (layer "B.Cu") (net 5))
 (segment (start 146.2 57.7) (end 148.5 60) (width 0.8) (layer "B.Cu") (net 5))
 (segment (start 115.265 65.1) (end 115.316 65.151) (width 0.8) (layer "F.Cu") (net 7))
 (segment (start 116.891 65.1) (end 118.313 65.1) (width 0.8) (layer "F.Cu") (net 7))
 (segment (start 118.415 65.1) (end 120.5 65.1) (width 0.8) (layer "F.Cu") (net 7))
 (segment (start 116.84 65.151) (end 116.891 65.1) (width 0.8) (layer "F.Cu") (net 7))
 (segment (start 118.313 65.1) (end 118.364 65.151) (width 0.8) (layer "F.Cu") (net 7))
 (segment (start 116.789 65.1) (end 116.84 65.151) (width 0.8) (layer "F.Cu") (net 7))
 (segment (start 113.5 65.1) (end 115.265 65.1) (width 0.8) (layer "F.Cu") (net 7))
 (segment (start 115.316 65.151) (end 115.367 65.1) (width 0.8) (layer "F.Cu") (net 7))
 (segment (start 118.364 65.151) (end 118.415 65.1) (width 0.8) (layer "F.Cu") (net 7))
 (segment (start 115.367 65.1) (end 116.789 65.1) (width 0.8) (layer "F.Cu") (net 7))
 (via (at 116.84 65.151) (size 0.8) (drill 0.4) (layers "F.Cu" "B.Cu") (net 7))
 (via (at 118.364 65.151) (size 0.8) (drill 0.4) (layers "F.Cu" "B.Cu") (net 7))
 (via (at 115.316 65.151) (size 0.8) (drill 0.4) (layers "F.Cu" "B.Cu") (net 7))
 (segment (start 138.639466 67.3) (end 142.421966 63.5175) (width 0.8) (layer "B.Cu") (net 7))
 (segment (start 142.421966 63.5175) (end 143.3575 63.5175) (width 0.8) (layer "B.Cu") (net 7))
 (segment (start 129.192214 63.135) (end 129.778 63.720786) (width 0.8) (layer "B.Cu") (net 7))
 (segment (start 133.3 67.3) (end 138.639466 67.3) (width 0.8) (layer "B.Cu") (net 7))
 (segment (start 129.778 63.778) (end 133.3 67.3) (width 0.8) (layer "B.Cu") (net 7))
 (segment (start 129.778 63.720786) (end 129.778 63.778) (width 0.8) (layer "B.Cu") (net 7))
 (segment (start 120.38 63.135) (end 129.192214 63.135) (width 0.8) (layer "B.Cu") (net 7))
 (segment (start 115.316 65.151) (end 118.364 65.151) (width 0.8) (layer "B.Cu") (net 7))
 (segment (start 118.364 65.151) (end 120.38 63.135) (width 0.8) (layer "B.Cu") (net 7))
 (segment (start 118.399 62.9) (end 118.364 62.865) (width 0.8) (layer "F.Cu") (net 6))
 (segment (start 116.875 62.9) (end 116.84 62.865) (width 0.8) (layer "F.Cu") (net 6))
 (segment (start 118.364 62.865) (end 118.329 62.9) (width 0.8) (layer "F.Cu") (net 6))
 (segment (start 115.316 62.865) (end 115.281 62.9) (width 0.8) (layer "F.Cu") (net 6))
 (segment (start 116.805 62.9) (end 115.351 62.9) (width 0.8) (layer "F.Cu") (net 6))
 (segment (start 120.5 62.9) (end 118.399 62.9) (width 0.8) (layer "F.Cu") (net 6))
 (segment (start 115.351 62.9) (end 115.316 62.865) (width 0.8) (layer "F.Cu") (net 6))
 (segment (start 118.329 62.9) (end 116.875 62.9) (width 0.8) (layer "F.Cu") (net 6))
 (segment (start 115.281 62.9) (end 113.5 62.9) (width 0.8) (layer "F.Cu") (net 6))
 (segment (start 116.84 62.865) (end 116.805 62.9) (width 0.8) (layer "F.Cu") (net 6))
 (via (at 116.84 62.865) (size 0.8) (drill 0.4) (layers "F.Cu" "B.Cu") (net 6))
 (via (at 118.364 62.865) (size 0.8) (drill 0.4) (layers "F.Cu" "B.Cu") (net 6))
 (via (at 115.316 62.865) (size 0.8) (drill 0.4) (layers "F.Cu" "B.Cu") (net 6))
 (segment (start 142.04 58.7) (end 143.3575 60.0175) (width 0.8) (layer "B.Cu") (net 6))
 (segment (start 130.662393 60.976) (end 132.938393 58.7) (width 0.8) (layer "B.Cu") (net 6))
 (segment (start 132.938393 58.7) (end 142.04 58.7) (width 0.8) (layer "B.Cu") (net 6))
 (segment (start 118.364 62.865) (end 120.253 60.976) (width 0.8) (layer "B.Cu") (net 6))
 (segment (start 120.253 60.976) (end 130.662393 60.976) (width 0.8) (layer "B.Cu") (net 6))
 (segment (start 115.316 62.865) (end 118.364 62.865) (width 0.8) (layer "B.Cu") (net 6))
 (segment (start 116.85 67.3) (end 118.354 67.3) (width 0.8) (layer "F.Cu") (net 8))
 (segment (start 116.84 67.31) (end 116.85 67.3) (width 0.8) (layer "F.Cu") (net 8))
 (segment (start 118.364 67.31) (end 118.374 67.3) (width 0.8) (layer "F.Cu") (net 8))
 (segment (start 115.316 67.31) (end 115.326 67.3) (width 0.8) (layer "F.Cu") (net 8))
 (segment (start 118.354 67.3) (end 118.364 67.31) (width 0.8) (layer "F.Cu") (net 8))
 (segment (start 116.83 67.3) (end 116.84 67.31) (width 0.8) (layer "F.Cu") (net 8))
 (segment (start 118.374 67.3) (end 120.5 67.3) (width 0.8) (layer "F.Cu") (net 8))
 (segment (start 113.5 67.3) (end 115.306 67.3) (width 0.8) (layer "F.Cu") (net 8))
 (segment (start 115.306 67.3) (end 115.316 67.31) (width 0.8) (layer "F.Cu") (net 8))
 (segment (start 115.326 67.3) (end 116.83 67.3) (width 0.8) (layer "F.Cu") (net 8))
 (via (at 115.316 67.31) (size 0.8) (drill 0.4) (layers "F.Cu" "B.Cu") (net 8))
 (via (at 116.84 67.31) (size 0.8) (drill 0.4) (layers "F.Cu" "B.Cu") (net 8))
 (via (at 118.364 67.31) (size 0.8) (drill 0.4) (layers "F.Cu" "B.Cu") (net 8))
 (segment (start 120.963 67.75) (end 120.523 67.31) (width 0.8) (layer "B.Cu") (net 8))
 (segment (start 141.075 69.3) (end 129.05 69.3) (width 0.8) (layer "B.Cu") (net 8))
 (segment (start 127.5 67.75) (end 120.963 67.75) (width 0.8) (layer "B.Cu") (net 8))
 (segment (start 129.05 69.3) (end 127.5 67.75) (width 0.8) (layer "B.Cu") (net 8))
 (segment (start 143.3575 67.0175) (end 141.075 69.3) (width 0.8) (layer "B.Cu") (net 8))
 (segment (start 120.523 67.31) (end 115.316 67.31) (width 0.8) (layer "B.Cu") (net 8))
 (segment (start 121.793 64.008) (end 112.703932 64.008) (width 0.3) (layer "F.Cu") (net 10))
 (segment (start 110.998 65.713932) (end 110.998 66.214) (width 0.3) (layer "F.Cu") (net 10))
 (segment (start 112.703932 64.008) (end 110.998 65.713932) (width 0.3) (layer "F.Cu") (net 10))
 (segment (start 123.063 65.278) (end 121.793 64.008) (width 0.3) (layer "F.Cu") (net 10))
 (segment (start 128.397 65.278) (end 123.063 65.278) (width 0.3) (layer "F.Cu") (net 10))
 (segment (start 130.419 67.3) (end 128.397 65.278) (width 0.3) (layer "F.Cu") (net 10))
 (segment (start 131 67.3) (end 130.419 67.3) (width 0.3) (layer "F.Cu") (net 10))
 (segment (start 112.1075 59.7) (end 110.998 60.8095) (width 0.3) (layer "F.Cu") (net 1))
 (segment (start 113.5 59.7) (end 112.1075 59.7) (width 0.3) (layer "F.Cu") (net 1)))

